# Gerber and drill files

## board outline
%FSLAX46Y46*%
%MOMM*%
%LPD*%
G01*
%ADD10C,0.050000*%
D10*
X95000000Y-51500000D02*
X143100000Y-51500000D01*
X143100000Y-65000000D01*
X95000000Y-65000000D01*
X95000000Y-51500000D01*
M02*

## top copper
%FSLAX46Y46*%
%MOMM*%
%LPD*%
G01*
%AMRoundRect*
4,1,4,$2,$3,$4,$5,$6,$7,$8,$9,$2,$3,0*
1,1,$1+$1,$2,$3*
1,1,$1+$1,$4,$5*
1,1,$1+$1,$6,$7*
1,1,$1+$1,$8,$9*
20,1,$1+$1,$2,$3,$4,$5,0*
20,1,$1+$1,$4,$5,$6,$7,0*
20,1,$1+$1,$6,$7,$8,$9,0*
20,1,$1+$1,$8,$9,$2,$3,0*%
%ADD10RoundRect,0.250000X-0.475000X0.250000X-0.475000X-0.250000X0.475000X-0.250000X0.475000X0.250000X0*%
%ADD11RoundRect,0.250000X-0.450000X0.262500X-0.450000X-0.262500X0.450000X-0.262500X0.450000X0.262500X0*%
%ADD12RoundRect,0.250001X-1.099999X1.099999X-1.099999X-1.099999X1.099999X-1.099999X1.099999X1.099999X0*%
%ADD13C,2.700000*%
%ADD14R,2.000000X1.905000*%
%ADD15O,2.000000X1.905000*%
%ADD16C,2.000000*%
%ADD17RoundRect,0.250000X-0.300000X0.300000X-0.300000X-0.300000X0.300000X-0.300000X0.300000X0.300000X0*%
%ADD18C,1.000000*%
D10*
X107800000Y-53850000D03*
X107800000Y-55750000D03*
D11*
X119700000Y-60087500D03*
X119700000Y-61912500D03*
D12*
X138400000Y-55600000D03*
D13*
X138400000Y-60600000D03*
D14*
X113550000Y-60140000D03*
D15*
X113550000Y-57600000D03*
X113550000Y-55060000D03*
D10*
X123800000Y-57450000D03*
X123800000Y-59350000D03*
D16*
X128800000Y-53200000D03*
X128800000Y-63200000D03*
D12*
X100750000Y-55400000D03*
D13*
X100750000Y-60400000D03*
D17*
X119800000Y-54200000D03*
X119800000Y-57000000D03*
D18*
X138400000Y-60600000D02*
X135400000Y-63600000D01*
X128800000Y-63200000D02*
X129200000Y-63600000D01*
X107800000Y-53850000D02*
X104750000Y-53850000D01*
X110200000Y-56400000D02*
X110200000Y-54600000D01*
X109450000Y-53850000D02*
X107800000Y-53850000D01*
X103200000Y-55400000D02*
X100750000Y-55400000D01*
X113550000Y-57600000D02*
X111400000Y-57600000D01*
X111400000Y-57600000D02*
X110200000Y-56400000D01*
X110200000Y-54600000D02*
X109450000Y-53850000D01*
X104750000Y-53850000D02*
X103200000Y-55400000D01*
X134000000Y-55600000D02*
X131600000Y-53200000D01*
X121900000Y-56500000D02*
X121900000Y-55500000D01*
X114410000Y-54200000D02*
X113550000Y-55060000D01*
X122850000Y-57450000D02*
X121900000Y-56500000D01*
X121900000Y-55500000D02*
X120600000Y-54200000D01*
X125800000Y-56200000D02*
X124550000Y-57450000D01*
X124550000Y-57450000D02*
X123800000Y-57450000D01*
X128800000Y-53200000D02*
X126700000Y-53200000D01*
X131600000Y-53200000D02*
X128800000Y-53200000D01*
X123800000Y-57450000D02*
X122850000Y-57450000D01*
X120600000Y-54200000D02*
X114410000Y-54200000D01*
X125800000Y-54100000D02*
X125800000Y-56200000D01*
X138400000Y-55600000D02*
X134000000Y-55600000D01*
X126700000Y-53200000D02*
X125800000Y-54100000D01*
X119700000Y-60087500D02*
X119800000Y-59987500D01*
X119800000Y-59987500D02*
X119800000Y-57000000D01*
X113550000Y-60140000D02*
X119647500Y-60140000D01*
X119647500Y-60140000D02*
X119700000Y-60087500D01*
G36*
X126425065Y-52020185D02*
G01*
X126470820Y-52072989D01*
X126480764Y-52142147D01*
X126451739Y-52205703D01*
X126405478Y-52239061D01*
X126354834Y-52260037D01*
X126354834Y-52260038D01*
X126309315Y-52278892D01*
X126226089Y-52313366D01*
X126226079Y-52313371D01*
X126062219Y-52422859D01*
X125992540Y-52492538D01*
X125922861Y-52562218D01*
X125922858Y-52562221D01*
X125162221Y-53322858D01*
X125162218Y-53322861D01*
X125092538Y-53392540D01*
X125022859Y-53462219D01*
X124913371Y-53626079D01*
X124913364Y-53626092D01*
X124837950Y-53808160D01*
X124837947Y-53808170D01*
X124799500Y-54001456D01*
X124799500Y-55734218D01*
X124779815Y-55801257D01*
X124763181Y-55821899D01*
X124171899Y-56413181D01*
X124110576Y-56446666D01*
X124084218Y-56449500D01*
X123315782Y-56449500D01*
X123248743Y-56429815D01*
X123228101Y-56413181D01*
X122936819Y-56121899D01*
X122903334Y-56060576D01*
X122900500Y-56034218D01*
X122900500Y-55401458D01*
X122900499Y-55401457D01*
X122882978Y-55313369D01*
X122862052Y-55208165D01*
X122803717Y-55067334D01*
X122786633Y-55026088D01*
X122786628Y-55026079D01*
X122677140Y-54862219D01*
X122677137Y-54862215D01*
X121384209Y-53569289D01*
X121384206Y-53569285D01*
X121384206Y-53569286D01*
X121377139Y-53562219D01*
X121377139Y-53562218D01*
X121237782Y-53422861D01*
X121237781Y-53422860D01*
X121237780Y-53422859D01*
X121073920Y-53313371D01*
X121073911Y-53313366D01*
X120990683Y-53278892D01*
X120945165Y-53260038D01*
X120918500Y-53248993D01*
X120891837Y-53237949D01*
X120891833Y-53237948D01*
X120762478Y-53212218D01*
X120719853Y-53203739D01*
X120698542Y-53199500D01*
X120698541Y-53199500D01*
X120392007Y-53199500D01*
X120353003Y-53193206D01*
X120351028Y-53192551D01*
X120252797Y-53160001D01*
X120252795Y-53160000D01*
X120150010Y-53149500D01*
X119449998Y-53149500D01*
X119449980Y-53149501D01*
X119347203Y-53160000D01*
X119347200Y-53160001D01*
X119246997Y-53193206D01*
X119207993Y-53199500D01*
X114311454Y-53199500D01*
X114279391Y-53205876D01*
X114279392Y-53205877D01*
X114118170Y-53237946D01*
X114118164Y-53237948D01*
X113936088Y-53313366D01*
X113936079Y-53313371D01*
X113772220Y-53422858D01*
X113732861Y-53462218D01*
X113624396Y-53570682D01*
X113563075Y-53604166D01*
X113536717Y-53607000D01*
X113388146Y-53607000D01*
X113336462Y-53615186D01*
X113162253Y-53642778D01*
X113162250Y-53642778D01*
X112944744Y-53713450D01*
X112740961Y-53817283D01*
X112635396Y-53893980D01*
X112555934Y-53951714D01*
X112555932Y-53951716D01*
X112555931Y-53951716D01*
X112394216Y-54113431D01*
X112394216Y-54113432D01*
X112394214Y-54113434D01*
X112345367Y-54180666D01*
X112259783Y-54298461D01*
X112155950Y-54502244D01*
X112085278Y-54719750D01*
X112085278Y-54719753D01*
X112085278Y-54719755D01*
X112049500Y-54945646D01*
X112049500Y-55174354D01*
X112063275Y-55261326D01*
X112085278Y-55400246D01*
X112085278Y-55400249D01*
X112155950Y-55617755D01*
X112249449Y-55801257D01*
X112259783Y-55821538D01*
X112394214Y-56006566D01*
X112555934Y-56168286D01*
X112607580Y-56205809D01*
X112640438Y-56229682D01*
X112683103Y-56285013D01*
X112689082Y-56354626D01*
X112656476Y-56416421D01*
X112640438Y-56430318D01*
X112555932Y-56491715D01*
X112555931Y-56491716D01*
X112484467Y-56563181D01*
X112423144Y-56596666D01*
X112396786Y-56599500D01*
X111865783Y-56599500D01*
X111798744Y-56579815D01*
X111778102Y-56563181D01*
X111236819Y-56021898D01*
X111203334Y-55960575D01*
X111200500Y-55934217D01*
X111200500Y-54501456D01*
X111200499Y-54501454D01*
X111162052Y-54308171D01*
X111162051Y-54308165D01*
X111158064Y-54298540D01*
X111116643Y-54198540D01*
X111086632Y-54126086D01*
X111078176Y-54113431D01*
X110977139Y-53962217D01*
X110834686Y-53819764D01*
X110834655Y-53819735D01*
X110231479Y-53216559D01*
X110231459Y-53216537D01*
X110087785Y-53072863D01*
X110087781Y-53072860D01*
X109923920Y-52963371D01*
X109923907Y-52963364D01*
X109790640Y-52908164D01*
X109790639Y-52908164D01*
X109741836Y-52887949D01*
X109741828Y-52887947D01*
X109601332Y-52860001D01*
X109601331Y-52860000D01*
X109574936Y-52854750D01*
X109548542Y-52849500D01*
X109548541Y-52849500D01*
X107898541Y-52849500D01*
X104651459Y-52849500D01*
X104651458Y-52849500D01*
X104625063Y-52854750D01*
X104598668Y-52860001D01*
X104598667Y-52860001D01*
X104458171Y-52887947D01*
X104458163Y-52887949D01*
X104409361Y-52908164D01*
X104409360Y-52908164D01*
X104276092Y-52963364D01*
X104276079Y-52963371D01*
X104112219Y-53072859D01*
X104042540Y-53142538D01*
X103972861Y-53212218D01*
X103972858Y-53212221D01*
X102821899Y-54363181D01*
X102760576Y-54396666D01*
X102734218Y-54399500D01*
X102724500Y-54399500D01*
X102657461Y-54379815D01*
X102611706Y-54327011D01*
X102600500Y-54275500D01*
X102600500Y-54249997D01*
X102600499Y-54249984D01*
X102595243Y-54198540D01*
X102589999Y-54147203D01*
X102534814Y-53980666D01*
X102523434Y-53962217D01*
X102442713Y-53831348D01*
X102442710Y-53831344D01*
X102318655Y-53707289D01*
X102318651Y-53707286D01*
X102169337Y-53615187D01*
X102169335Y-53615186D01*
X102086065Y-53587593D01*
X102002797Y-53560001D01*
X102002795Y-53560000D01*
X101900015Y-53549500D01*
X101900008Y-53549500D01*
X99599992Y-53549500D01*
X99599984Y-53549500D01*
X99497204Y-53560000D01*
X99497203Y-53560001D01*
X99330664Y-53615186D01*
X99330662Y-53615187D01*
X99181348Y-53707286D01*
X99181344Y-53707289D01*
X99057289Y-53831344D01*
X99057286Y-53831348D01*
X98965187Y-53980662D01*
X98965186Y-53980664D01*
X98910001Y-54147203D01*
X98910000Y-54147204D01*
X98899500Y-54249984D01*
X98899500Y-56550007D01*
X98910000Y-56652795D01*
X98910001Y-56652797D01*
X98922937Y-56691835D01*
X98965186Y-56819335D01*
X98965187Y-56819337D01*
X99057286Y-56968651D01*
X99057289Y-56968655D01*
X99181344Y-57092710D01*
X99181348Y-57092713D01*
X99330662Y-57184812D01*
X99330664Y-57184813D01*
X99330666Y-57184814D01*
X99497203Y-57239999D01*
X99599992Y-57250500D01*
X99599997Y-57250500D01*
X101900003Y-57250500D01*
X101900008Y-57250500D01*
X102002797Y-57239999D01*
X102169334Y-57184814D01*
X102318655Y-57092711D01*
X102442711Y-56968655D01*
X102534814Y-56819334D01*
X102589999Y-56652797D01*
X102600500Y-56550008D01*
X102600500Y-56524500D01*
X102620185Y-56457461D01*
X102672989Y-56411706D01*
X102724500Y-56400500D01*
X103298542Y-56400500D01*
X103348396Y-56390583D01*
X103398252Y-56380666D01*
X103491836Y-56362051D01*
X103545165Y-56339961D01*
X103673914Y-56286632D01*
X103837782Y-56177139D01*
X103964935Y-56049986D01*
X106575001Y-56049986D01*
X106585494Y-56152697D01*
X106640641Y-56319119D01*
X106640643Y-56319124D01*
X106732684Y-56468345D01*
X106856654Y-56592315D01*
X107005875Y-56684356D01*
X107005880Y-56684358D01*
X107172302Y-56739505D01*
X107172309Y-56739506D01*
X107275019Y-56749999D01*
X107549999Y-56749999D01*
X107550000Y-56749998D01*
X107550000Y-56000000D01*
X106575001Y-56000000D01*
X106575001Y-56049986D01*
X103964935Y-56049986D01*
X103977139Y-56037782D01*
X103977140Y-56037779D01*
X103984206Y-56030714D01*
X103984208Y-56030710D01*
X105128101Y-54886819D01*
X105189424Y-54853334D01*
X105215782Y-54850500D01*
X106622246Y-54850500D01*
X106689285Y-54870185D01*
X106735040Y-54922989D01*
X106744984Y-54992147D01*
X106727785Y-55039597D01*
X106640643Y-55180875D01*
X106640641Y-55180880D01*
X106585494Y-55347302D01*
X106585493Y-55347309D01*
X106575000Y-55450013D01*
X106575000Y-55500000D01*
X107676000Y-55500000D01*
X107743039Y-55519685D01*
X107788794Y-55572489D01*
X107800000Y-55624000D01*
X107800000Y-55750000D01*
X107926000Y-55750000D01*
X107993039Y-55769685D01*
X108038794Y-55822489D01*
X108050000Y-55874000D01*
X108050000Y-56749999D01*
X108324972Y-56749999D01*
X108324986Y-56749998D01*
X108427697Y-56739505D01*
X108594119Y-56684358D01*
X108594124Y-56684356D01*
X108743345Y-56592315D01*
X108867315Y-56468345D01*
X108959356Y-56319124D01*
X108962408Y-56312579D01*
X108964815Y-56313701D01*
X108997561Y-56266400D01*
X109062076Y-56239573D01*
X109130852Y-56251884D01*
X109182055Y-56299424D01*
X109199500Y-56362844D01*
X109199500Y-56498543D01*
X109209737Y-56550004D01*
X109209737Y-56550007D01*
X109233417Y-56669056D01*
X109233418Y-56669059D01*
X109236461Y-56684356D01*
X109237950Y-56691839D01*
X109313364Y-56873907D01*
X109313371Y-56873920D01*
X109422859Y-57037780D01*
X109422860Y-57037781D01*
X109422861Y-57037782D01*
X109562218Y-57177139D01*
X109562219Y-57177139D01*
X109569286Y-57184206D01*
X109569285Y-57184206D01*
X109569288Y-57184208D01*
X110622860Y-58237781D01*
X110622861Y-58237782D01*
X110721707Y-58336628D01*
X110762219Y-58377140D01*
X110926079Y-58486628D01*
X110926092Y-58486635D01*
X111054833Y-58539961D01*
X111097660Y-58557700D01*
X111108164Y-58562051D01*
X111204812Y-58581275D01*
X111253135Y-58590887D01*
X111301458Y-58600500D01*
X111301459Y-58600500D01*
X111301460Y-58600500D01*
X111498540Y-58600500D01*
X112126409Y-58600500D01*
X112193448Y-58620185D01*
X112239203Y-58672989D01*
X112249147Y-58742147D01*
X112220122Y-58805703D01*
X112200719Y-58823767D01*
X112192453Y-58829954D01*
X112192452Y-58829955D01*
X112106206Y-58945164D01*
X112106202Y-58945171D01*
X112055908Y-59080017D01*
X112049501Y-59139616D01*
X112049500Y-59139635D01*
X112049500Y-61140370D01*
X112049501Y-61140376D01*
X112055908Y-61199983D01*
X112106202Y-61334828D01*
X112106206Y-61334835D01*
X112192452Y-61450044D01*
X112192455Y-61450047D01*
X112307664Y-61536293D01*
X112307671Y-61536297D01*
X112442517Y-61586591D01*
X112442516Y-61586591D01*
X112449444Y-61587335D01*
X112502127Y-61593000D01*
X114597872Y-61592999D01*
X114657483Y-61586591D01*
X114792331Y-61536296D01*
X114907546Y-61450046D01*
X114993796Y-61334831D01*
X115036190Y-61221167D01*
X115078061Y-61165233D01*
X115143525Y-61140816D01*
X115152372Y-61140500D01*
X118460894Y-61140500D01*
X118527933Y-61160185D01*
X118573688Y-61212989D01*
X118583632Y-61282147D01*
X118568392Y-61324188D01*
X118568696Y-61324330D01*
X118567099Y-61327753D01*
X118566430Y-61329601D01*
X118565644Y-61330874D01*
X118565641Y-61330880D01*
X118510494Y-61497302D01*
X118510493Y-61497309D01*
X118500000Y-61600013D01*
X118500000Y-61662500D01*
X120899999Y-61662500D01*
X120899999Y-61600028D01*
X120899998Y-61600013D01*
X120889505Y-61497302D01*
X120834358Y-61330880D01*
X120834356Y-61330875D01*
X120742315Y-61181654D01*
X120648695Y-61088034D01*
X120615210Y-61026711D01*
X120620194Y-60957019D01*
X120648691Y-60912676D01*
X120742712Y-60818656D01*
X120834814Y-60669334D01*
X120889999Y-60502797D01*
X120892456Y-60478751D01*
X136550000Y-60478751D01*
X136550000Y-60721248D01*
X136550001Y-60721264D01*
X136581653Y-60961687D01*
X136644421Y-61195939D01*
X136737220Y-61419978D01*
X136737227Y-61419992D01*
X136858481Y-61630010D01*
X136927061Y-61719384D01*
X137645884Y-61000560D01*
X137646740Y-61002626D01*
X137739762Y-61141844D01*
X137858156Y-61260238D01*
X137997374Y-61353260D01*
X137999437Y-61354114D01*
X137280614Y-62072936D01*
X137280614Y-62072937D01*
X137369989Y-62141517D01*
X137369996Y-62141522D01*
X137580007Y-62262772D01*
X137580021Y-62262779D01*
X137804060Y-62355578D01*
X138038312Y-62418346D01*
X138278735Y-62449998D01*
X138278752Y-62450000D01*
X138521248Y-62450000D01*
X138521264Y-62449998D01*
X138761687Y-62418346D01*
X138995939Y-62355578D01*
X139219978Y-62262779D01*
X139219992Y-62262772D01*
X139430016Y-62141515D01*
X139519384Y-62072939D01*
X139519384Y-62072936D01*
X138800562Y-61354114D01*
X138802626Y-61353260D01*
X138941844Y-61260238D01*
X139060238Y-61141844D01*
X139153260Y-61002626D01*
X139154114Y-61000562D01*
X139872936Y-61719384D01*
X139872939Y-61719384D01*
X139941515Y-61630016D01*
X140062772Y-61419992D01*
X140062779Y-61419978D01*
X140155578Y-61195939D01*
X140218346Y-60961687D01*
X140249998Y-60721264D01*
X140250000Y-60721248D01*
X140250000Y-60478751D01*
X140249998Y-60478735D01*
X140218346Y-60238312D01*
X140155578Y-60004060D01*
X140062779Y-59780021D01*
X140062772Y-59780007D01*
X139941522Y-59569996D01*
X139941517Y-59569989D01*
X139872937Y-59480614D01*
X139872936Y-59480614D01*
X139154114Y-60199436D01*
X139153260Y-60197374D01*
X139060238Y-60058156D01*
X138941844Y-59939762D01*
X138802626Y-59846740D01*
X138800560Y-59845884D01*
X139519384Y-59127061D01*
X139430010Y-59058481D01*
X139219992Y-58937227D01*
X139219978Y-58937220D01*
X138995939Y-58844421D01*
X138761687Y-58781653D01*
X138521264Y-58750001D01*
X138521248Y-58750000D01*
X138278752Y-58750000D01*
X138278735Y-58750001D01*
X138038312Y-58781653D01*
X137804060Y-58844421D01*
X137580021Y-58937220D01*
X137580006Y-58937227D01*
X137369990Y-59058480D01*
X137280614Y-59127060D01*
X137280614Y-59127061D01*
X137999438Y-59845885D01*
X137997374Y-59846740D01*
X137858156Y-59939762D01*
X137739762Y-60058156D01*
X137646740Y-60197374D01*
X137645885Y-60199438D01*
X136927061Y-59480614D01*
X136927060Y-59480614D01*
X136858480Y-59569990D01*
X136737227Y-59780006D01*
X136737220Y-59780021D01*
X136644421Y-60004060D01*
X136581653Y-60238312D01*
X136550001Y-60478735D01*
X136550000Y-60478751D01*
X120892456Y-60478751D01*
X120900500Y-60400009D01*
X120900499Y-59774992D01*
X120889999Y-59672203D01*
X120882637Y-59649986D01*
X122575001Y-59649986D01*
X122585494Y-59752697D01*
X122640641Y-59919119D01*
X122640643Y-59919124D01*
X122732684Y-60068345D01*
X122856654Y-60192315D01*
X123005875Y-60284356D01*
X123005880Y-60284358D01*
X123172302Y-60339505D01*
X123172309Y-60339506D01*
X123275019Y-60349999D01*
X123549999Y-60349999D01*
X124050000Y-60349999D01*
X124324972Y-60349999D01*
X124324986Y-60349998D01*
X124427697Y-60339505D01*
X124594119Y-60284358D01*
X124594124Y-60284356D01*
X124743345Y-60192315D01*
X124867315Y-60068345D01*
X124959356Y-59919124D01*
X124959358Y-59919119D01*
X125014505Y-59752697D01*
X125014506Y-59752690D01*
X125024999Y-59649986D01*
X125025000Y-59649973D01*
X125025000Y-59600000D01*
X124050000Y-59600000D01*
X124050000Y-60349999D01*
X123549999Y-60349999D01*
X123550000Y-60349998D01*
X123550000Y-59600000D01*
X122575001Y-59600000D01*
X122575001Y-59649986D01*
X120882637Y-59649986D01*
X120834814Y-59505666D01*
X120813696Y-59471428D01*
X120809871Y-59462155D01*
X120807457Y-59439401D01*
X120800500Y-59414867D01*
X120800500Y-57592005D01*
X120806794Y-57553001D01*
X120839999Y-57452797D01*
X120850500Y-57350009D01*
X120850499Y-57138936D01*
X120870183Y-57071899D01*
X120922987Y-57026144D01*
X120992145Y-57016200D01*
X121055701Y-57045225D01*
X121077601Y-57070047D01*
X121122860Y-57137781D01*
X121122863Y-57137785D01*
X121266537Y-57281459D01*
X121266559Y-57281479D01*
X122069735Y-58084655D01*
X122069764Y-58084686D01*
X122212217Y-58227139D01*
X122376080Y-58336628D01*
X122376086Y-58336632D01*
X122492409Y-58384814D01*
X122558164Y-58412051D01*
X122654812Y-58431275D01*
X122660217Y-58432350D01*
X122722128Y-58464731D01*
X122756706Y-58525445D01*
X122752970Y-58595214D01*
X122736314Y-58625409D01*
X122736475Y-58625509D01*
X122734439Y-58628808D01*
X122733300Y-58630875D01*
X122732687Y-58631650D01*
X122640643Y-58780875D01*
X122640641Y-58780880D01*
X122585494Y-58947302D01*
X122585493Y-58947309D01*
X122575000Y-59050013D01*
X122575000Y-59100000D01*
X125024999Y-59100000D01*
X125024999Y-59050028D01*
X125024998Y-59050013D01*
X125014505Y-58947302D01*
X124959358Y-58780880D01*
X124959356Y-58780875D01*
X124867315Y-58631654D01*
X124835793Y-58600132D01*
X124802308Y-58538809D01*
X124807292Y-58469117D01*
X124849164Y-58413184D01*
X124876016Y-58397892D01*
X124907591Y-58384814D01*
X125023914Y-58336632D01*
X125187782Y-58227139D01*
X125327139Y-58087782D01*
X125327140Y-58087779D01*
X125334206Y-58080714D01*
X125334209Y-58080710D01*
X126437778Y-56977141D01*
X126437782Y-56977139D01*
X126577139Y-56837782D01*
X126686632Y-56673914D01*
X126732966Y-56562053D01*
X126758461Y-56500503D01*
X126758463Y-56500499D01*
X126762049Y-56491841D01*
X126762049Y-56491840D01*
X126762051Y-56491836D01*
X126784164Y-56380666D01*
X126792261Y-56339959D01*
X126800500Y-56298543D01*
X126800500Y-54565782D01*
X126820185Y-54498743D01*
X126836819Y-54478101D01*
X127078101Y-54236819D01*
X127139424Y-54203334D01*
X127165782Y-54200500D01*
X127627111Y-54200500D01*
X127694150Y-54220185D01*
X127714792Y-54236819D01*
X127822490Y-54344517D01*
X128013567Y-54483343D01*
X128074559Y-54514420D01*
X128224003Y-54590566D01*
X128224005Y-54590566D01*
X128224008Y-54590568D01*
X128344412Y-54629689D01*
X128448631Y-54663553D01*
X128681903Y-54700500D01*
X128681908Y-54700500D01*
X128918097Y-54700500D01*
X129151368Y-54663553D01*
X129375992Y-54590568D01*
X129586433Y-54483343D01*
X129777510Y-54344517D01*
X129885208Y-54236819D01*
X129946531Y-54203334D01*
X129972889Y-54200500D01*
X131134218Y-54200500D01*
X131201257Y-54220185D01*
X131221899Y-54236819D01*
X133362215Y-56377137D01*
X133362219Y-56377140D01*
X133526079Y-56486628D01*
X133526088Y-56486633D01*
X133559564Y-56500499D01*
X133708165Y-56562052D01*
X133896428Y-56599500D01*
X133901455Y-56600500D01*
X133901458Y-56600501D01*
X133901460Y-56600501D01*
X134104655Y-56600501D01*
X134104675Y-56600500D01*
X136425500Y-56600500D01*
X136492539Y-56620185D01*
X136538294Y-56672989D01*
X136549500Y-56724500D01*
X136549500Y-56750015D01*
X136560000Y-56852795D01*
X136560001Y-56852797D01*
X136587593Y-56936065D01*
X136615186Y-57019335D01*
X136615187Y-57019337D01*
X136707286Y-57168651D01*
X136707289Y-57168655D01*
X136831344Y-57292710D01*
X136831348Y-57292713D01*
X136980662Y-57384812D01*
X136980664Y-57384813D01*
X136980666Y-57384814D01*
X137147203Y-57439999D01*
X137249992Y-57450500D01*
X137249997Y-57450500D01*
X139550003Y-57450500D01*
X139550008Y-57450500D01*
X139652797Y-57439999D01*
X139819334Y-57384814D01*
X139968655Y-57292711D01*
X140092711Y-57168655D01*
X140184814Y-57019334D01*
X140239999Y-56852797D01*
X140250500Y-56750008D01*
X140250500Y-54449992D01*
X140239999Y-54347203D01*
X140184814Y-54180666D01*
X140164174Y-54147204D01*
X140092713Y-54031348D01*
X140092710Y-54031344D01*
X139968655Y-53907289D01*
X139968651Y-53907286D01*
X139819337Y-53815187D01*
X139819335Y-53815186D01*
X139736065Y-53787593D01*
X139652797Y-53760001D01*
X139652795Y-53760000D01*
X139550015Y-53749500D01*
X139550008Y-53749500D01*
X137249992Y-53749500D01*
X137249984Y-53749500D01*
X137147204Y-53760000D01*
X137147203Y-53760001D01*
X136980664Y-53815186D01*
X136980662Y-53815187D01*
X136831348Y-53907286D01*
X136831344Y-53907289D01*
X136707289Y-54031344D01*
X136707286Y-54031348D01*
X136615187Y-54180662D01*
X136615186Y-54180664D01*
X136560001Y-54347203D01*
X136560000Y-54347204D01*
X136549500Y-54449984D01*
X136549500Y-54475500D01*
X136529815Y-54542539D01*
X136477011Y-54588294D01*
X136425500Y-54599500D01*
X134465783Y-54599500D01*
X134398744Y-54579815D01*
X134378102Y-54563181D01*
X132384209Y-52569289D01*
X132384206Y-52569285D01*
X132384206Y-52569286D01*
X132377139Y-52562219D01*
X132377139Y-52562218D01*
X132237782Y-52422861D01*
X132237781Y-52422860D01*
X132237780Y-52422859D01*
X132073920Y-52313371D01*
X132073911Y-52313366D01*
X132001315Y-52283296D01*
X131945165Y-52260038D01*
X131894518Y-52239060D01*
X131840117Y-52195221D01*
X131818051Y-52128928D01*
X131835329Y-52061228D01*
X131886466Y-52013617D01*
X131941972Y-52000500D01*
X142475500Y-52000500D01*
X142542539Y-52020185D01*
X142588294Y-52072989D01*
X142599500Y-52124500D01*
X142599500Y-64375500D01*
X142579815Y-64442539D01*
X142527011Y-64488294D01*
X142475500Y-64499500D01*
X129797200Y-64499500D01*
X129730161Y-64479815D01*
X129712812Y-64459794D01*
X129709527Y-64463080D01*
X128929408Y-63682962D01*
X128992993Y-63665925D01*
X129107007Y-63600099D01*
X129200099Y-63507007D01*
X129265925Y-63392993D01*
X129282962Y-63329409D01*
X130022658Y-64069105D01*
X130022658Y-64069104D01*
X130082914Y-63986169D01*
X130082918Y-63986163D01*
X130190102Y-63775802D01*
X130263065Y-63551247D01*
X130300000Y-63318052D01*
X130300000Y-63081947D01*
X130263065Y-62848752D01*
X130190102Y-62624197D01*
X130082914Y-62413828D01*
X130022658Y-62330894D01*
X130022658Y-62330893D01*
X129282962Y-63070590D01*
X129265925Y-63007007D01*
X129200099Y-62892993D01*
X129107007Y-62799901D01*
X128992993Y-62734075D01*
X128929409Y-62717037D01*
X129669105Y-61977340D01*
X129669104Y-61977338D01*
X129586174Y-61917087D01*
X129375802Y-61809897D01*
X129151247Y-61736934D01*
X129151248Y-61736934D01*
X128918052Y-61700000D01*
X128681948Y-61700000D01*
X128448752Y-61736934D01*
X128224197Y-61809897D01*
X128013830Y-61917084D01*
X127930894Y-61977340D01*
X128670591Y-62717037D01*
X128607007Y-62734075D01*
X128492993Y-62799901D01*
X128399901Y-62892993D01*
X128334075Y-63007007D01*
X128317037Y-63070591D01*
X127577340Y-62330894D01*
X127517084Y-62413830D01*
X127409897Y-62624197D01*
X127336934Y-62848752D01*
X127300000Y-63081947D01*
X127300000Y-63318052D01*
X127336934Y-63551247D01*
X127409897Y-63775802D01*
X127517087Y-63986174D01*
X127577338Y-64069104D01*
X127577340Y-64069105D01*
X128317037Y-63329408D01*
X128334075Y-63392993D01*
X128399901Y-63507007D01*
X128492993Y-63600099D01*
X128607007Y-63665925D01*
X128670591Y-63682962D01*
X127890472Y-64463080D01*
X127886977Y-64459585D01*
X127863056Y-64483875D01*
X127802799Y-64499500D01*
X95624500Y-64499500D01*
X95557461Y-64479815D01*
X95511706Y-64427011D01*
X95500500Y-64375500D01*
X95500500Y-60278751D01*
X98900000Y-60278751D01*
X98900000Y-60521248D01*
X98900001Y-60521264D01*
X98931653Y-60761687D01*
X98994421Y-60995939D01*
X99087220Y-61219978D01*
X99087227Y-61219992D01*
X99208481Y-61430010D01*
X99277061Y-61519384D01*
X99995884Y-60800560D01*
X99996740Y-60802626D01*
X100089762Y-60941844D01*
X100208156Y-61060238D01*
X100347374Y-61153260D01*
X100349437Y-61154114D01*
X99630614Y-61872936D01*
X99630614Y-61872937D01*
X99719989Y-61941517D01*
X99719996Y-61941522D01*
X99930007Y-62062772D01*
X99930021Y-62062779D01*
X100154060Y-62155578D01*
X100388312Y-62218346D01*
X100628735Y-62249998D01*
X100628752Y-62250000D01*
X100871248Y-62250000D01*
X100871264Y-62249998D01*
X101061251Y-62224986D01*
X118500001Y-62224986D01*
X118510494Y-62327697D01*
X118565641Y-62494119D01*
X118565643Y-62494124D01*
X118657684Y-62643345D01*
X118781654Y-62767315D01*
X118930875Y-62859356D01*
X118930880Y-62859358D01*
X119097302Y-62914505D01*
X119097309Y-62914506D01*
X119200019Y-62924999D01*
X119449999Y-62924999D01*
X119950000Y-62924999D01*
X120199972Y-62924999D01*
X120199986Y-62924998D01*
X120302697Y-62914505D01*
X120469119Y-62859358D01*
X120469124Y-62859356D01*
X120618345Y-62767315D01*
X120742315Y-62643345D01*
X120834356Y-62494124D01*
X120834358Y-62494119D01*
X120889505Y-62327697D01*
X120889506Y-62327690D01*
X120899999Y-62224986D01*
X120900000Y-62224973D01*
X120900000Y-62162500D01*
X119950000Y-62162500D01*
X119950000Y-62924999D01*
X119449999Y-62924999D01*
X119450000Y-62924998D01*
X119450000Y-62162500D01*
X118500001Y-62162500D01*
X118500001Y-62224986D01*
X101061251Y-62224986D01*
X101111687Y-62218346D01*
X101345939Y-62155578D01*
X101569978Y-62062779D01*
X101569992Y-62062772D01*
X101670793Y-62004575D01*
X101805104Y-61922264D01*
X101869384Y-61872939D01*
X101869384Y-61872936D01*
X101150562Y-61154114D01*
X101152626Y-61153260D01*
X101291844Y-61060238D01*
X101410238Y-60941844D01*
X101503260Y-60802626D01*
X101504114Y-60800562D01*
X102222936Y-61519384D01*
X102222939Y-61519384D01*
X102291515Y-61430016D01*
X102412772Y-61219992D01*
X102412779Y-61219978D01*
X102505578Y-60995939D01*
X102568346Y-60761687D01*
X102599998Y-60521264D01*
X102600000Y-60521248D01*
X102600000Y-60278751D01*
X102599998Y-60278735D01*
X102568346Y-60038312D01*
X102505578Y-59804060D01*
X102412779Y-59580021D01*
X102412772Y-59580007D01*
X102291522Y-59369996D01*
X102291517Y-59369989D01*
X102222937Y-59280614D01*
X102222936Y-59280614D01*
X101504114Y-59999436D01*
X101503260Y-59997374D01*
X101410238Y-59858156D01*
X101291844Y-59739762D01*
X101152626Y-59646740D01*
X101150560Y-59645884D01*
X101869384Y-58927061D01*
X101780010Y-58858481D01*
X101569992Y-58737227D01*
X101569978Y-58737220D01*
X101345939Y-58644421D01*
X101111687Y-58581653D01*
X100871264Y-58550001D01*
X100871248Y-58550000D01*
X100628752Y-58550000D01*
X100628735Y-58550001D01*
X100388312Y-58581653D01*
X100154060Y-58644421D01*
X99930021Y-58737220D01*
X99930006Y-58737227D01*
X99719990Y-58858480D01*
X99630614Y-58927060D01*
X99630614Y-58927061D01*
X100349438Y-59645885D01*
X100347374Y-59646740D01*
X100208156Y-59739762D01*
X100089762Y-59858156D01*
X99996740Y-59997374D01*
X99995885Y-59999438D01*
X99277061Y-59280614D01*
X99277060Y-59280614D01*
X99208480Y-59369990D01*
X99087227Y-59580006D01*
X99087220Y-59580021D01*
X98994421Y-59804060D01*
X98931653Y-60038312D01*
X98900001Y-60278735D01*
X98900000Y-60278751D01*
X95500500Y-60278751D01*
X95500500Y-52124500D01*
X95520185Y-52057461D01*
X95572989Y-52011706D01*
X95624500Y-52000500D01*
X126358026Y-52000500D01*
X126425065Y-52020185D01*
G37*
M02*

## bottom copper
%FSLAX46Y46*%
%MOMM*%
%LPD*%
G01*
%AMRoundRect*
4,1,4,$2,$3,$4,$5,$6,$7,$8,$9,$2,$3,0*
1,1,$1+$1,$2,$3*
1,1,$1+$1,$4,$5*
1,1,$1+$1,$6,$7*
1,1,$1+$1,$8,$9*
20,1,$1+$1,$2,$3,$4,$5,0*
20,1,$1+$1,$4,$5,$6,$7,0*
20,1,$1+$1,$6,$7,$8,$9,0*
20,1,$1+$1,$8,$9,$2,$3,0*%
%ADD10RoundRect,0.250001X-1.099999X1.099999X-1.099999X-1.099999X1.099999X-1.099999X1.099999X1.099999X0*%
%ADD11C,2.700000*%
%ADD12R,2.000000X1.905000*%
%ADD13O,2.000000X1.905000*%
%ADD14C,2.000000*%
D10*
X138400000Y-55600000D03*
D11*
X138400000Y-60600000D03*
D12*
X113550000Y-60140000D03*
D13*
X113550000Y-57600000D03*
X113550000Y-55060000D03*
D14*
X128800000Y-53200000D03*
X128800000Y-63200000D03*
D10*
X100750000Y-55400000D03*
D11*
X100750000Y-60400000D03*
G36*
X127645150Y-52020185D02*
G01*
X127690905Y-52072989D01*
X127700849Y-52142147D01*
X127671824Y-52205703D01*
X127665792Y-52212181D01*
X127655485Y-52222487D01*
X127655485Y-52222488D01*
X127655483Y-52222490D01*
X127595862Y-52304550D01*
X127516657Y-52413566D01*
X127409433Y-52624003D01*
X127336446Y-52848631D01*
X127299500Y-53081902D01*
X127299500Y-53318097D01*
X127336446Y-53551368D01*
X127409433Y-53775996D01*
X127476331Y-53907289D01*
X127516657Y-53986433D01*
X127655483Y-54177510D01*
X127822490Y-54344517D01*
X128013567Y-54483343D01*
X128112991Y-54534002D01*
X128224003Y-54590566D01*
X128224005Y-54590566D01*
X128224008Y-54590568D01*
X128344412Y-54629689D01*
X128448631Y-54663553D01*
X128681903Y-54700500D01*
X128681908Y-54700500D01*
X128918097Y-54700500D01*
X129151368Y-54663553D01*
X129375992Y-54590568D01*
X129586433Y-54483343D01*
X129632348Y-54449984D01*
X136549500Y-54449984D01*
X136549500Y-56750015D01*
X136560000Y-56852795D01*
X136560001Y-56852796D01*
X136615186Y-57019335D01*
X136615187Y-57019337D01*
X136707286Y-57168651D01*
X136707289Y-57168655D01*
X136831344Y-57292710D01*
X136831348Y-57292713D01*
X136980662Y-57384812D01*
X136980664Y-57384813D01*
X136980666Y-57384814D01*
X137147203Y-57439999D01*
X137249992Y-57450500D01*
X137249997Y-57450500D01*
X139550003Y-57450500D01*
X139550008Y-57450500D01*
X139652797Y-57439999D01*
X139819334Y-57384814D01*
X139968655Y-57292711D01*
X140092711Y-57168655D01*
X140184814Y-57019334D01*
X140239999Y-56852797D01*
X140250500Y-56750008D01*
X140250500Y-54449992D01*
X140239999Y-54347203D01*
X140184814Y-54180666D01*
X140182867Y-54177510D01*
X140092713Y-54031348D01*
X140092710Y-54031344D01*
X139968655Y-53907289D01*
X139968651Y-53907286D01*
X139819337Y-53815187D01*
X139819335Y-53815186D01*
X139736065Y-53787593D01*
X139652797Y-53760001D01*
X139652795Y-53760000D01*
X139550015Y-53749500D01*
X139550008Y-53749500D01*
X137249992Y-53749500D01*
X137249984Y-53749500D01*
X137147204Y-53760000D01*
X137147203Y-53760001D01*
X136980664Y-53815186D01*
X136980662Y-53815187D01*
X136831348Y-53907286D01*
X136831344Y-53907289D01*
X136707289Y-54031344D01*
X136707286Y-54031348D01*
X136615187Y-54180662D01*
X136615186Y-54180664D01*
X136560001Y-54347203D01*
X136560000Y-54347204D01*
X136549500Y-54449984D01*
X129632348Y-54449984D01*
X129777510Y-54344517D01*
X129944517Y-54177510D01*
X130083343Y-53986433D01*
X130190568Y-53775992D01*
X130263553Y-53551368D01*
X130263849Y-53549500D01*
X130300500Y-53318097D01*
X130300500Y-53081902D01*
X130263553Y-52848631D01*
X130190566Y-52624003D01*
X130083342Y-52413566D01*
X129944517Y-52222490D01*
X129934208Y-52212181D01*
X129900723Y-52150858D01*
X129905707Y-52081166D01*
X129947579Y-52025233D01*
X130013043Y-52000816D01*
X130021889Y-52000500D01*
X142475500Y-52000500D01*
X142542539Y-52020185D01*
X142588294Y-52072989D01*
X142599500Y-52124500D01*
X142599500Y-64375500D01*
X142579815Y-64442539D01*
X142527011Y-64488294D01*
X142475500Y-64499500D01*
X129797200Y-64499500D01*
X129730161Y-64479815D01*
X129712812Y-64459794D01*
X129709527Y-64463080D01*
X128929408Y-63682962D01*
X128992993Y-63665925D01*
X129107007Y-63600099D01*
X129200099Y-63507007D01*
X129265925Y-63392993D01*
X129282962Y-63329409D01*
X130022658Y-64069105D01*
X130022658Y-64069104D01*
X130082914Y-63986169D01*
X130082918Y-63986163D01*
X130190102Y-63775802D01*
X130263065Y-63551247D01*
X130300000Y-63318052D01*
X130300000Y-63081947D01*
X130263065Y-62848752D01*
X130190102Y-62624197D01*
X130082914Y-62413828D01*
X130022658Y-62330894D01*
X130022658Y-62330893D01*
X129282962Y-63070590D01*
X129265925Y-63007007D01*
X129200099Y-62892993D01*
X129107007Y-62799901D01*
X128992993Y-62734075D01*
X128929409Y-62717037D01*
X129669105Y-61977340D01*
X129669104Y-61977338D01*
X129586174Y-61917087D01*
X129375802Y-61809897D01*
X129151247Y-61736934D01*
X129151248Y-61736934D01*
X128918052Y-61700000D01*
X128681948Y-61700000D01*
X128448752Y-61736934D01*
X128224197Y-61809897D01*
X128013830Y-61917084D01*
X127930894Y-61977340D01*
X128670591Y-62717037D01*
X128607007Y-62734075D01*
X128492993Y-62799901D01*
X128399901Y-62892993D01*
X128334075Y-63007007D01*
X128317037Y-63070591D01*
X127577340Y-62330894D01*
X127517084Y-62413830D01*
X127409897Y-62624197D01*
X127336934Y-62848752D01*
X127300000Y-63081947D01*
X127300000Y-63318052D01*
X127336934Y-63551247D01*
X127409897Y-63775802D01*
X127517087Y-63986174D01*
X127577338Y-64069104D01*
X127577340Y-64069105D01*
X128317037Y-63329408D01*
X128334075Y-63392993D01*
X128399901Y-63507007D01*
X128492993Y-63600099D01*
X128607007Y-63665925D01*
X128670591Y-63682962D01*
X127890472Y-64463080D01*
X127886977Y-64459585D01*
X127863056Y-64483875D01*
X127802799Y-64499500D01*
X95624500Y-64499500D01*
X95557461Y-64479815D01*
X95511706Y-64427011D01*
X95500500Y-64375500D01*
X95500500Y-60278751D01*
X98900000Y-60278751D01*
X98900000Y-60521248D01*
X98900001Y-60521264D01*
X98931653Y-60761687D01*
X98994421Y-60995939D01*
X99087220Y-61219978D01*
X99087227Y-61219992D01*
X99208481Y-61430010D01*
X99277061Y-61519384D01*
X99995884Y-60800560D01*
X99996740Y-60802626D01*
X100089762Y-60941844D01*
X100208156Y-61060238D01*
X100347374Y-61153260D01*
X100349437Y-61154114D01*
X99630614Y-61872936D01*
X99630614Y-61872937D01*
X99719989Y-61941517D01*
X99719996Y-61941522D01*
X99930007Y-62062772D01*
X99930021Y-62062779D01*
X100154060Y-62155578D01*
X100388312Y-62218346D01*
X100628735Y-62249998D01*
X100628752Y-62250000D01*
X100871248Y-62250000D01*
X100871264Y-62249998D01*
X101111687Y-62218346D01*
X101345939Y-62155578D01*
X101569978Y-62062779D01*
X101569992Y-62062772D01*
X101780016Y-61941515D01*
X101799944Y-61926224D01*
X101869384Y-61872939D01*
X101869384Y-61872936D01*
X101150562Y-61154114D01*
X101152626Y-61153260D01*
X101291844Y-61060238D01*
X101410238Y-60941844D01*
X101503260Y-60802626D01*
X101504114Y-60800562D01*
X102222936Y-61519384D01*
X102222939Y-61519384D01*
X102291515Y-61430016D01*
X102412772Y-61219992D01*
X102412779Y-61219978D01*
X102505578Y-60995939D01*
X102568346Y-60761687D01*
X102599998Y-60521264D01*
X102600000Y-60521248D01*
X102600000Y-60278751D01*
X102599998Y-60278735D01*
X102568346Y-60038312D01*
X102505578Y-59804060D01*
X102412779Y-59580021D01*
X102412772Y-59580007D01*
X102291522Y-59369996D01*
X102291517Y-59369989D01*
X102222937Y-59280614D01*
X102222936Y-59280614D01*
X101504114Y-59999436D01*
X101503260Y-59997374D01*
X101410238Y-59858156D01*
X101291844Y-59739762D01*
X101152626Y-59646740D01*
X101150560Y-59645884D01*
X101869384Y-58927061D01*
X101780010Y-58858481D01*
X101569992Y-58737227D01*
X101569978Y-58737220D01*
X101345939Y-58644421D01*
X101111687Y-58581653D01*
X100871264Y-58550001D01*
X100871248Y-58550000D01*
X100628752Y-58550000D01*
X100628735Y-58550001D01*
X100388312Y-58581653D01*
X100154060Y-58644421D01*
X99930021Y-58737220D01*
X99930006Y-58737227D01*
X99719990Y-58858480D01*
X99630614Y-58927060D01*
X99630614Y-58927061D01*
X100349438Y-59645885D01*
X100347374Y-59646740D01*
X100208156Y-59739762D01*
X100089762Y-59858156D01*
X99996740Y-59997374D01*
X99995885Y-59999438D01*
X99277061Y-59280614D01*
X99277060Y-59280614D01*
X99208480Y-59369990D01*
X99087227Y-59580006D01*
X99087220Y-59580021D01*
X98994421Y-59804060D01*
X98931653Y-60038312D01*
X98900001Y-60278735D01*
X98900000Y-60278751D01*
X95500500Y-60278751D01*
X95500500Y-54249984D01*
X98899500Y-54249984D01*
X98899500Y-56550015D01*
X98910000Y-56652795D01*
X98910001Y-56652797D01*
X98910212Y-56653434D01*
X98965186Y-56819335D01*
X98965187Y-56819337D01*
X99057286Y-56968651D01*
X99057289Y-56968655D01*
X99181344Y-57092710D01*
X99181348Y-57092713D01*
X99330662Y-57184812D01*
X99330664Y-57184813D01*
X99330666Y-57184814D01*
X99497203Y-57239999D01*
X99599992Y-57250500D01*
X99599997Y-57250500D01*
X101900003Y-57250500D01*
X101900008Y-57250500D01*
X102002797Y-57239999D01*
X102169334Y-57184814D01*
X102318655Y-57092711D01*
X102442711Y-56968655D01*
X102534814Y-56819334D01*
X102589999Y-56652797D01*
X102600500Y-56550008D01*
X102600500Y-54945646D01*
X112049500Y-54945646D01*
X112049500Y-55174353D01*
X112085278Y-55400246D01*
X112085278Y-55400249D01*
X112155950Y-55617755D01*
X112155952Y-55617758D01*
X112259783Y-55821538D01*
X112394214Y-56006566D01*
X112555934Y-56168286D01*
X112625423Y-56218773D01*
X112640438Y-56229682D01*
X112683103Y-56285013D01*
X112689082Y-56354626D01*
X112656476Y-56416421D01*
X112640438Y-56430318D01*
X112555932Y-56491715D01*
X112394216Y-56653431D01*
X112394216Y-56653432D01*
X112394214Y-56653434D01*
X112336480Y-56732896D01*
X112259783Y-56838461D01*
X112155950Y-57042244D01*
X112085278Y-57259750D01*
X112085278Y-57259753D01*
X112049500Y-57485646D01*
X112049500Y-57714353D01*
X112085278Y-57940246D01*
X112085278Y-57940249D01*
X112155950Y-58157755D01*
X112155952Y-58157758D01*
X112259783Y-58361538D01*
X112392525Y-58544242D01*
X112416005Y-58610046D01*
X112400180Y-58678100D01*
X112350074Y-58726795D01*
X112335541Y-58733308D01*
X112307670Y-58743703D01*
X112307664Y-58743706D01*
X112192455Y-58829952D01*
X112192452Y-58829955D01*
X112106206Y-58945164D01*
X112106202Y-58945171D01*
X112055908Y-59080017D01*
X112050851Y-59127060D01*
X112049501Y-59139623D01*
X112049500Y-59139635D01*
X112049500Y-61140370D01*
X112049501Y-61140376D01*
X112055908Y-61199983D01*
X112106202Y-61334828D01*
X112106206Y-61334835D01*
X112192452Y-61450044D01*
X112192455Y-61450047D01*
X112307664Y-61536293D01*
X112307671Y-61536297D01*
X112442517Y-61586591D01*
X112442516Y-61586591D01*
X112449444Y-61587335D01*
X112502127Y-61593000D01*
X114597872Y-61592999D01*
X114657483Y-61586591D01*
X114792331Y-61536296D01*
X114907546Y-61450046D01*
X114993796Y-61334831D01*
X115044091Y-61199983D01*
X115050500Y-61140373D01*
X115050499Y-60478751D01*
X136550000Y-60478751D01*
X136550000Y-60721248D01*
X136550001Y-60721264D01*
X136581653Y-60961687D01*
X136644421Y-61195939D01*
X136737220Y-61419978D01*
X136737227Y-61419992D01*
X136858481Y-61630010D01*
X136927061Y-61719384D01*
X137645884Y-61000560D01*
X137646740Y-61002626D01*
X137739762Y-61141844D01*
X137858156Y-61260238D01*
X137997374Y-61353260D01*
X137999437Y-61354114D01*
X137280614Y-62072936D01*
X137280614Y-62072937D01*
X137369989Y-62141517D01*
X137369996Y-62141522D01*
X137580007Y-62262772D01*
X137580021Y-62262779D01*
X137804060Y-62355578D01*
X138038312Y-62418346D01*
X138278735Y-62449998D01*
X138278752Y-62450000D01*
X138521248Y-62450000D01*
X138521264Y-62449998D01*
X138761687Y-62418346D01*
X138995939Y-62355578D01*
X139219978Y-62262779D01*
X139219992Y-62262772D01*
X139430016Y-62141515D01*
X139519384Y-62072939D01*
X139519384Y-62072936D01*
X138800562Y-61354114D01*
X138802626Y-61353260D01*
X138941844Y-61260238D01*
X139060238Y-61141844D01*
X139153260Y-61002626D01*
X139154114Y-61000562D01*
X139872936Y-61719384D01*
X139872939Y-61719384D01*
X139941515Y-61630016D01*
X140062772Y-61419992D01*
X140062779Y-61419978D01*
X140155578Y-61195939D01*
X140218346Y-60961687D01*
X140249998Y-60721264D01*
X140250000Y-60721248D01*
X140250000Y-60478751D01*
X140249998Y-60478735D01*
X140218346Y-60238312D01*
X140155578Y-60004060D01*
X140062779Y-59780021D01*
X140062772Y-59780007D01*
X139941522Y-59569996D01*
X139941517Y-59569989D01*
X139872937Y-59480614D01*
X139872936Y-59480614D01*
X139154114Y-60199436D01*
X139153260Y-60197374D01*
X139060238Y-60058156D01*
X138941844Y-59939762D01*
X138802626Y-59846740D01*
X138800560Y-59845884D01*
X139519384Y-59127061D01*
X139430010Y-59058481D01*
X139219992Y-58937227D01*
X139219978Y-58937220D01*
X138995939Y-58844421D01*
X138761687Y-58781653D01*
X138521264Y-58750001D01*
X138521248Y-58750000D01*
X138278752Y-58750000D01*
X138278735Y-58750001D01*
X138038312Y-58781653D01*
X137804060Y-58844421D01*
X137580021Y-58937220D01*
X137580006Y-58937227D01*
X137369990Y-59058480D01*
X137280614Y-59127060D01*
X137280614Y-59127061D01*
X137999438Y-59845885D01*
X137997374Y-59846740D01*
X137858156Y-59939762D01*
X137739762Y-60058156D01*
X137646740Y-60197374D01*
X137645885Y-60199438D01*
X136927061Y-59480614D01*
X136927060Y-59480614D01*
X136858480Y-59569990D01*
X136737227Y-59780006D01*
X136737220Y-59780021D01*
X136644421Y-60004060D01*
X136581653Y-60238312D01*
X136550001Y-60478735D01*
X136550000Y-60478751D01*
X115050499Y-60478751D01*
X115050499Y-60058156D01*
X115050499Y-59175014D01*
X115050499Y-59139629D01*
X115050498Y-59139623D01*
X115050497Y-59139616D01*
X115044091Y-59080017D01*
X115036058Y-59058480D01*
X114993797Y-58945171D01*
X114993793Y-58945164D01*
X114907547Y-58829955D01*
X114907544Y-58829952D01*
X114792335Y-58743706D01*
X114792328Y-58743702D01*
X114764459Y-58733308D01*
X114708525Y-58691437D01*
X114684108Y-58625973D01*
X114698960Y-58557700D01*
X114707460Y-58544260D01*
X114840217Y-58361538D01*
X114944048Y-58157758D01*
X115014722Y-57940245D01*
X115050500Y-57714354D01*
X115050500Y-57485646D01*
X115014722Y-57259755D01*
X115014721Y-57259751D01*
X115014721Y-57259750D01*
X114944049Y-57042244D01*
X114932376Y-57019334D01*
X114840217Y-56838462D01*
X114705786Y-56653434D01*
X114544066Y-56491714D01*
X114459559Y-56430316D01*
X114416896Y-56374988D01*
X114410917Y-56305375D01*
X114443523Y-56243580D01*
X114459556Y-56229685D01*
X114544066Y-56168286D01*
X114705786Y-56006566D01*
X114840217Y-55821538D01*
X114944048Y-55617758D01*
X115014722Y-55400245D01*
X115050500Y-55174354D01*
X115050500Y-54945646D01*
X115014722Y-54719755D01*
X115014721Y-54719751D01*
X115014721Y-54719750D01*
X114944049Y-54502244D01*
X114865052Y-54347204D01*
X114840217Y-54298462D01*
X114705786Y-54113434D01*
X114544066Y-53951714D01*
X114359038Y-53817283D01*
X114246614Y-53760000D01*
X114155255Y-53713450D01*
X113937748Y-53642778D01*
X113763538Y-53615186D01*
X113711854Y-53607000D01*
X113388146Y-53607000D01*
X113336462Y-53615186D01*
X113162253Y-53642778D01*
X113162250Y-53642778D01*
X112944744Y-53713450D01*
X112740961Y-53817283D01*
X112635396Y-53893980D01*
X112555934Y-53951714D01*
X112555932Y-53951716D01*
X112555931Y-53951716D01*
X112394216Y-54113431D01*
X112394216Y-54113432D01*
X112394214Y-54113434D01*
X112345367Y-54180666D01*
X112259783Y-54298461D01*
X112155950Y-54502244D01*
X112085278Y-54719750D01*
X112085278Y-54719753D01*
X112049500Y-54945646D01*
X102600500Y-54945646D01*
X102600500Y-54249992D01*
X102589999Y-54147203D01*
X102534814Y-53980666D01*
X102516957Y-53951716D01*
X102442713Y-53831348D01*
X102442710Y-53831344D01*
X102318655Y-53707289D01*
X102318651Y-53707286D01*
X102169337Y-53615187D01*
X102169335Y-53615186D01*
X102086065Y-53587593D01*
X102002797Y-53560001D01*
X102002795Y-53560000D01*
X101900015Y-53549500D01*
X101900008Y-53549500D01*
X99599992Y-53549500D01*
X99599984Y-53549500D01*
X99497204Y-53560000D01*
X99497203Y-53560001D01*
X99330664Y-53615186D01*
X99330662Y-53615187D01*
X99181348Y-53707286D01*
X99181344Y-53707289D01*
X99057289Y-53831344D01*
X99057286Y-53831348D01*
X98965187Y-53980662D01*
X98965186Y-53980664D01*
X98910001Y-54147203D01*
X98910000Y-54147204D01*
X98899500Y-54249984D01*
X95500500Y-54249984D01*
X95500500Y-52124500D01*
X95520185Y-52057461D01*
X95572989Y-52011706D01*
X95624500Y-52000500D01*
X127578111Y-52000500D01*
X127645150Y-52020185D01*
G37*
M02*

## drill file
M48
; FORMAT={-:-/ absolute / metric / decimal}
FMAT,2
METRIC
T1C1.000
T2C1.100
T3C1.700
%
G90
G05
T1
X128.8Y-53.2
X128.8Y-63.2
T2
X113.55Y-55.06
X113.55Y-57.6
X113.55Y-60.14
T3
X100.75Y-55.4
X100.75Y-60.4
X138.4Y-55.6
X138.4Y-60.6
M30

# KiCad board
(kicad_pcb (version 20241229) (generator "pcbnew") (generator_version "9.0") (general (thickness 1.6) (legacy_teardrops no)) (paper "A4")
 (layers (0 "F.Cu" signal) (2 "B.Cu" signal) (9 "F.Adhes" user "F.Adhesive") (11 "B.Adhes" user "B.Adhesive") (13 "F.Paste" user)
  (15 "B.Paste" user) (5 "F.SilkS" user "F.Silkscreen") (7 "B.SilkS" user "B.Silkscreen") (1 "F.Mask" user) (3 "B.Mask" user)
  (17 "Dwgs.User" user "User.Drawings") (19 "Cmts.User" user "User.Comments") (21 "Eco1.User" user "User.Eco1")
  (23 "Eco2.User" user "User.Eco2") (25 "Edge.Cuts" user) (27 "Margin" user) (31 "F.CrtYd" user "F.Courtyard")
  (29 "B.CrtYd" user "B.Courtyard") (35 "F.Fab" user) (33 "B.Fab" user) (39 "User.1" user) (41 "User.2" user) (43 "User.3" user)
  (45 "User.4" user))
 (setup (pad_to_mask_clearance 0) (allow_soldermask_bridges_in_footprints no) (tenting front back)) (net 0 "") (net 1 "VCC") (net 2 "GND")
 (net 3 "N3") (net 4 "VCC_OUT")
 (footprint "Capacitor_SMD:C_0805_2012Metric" (layer "F.Cu") (at 107.8 54.8 -90)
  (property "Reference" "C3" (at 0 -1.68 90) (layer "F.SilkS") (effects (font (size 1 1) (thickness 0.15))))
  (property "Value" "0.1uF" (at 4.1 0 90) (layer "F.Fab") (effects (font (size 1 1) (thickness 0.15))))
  (pad "1" smd roundrect (at -0.95 0 270) (size 1 1.45) (layers "F.Cu" "F.Mask" "F.Paste") (roundrect_rratio 0.25) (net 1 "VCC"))
  (pad "2" smd roundrect (at 0.95 0 270) (size 1 1.45) (layers "F.Cu" "F.Mask" "F.Paste") (roundrect_rratio 0.25) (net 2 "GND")))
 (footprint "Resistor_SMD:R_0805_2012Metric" (layer "F.Cu") (at 119.7 61 -90)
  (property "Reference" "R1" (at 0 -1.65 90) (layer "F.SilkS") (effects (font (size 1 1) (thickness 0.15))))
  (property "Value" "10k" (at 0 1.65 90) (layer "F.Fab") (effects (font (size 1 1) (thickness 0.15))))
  (pad "1" smd roundrect (at -0.9125 0 270) (size 1.025 1.4) (layers "F.Cu" "F.Mask" "F.Paste") (roundrect_rratio 0.243902) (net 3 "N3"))
  (pad "2" smd roundrect (at 0.9125 0 270) (size 1.025 1.4) (layers "F.Cu" "F.Mask" "F.Paste") (roundrect_rratio 0.243902) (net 2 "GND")))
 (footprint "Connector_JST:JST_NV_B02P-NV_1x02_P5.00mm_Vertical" (layer "F.Cu") (at 138.4 55.6 -90)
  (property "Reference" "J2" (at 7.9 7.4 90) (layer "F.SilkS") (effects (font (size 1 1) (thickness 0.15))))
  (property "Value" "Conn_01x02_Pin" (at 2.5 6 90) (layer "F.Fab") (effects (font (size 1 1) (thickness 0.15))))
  (pad "1" thru_hole roundrect (at 0 0 270) (size 2.7 2.7) (drill 1.7) (layers "*.Cu" "*.Mask") (remove_unused_layers no)
   (roundrect_rratio 0.092593) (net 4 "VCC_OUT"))
  (pad "2" thru_hole circle (at 5 0 270) (size 2.7 2.7) (drill 1.7) (layers "*.Cu" "*.Mask") (remove_unused_layers no) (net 2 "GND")))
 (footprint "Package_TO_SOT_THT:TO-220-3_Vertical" (layer "F.Cu") (at 113.55 60.14 90)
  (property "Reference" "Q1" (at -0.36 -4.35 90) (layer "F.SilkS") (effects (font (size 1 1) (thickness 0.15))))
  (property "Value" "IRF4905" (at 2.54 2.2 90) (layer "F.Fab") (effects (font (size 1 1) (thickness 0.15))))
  (pad "1" thru_hole rect (at 0 0 90) (size 1.905 2) (drill 1.1) (layers "*.Cu" "*.Mask") (remove_unused_layers no) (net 3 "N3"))
  (pad "2" thru_hole oval (at 2.54 0 90) (size 1.905 2) (drill 1.1) (layers "*.Cu" "*.Mask") (remove_unused_layers no) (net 1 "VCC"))
  (pad "3" thru_hole oval (at 5.08 0 90) (size 1.905 2) (drill 1.1) (layers "*.Cu" "*.Mask") (remove_unused_layers no) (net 4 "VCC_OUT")))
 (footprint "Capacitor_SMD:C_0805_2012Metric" (layer "F.Cu") (at 123.8 58.4 -90)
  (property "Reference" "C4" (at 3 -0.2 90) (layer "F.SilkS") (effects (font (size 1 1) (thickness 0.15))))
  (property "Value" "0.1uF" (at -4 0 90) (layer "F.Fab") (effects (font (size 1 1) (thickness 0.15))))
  (pad "1" smd roundrect (at -0.95 0 270) (size 1 1.45) (layers "F.Cu" "F.Mask" "F.Paste") (roundrect_rratio 0.25) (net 4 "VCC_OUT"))
  (pad "2" smd roundrect (at 0.95 0 270) (size 1 1.45) (layers "F.Cu" "F.Mask" "F.Paste") (roundrect_rratio 0.25) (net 2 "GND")))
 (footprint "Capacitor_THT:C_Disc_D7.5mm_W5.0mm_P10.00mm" (layer "F.Cu") (at 128.8 53.2 -90)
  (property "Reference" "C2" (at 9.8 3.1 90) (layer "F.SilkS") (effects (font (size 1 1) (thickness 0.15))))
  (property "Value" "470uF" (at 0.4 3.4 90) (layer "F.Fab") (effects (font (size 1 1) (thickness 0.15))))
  (pad "1" thru_hole circle (at 0 0 270) (size 2 2) (drill 1) (layers "*.Cu" "*.Mask") (remove_unused_layers no) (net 4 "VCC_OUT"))
  (pad "2" thru_hole circle (at 10 0 270) (size 2 2) (drill 1) (layers "*.Cu" "*.Mask") (remove_unused_layers no) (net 2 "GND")))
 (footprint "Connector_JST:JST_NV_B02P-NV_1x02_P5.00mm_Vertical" (layer "F.Cu") (at 100.75 55.4 -90)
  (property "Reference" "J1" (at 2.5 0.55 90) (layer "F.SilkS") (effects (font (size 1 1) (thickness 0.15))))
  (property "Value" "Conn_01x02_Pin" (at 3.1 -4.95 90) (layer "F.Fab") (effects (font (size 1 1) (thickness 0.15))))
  (pad "1" thru_hole roundrect (at 0 0 270) (size 2.7 2.7) (drill 1.7) (layers "*.Cu" "*.Mask") (remove_unused_layers no)
   (roundrect_rratio 0.092593) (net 1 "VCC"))
  (pad "2" thru_hole circle (at 5 0 270) (size 2.7 2.7) (drill 1.7) (layers "*.Cu" "*.Mask") (remove_unused_layers no) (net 2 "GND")))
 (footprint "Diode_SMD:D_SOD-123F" (layer "F.Cu") (at 119.8 55.6 -90)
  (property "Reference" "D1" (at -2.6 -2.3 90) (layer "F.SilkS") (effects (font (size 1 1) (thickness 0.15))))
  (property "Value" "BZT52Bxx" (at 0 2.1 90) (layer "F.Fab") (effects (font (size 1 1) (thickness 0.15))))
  (pad "1" smd roundrect (at -1.4 0 270) (size 1.1 1.1) (layers "F.Cu" "F.Mask" "F.Paste") (roundrect_rratio 0.2272727273) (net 4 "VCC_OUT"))
  (pad "2" smd roundrect (at 1.4 0 270) (size 1.1 1.1) (layers "F.Cu" "F.Mask" "F.Paste") (roundrect_rratio 0.2272727273) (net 3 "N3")))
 (gr_rect (start 95 51.5) (end 143.1 65) (stroke (width 0.05) (type default)) (fill no) (layer "Edge.Cuts"))
 (segment (start 138.4 60.6) (end 135.4 63.6) (width 1) (layer "F.Cu") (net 2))
 (segment (start 128.8 63.2) (end 129.2 63.6) (width 1) (layer "F.Cu") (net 2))
 (segment (start 107.8 53.85) (end 104.75 53.85) (width 1) (layer "F.Cu") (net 1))
 (segment (start 110.2 56.4) (end 110.2 54.6) (width 1) (layer "F.Cu") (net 1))
 (segment (start 109.45 53.85) (end 107.8 53.85) (width 1) (layer "F.Cu") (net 1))
 (segment (start 103.2 55.4) (end 100.75 55.4) (width 1) (layer "F.Cu") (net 1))
 (segment (start 113.55 57.6) (end 111.4 57.6) (width 1) (layer "F.Cu") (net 1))
 (segment (start 111.4 57.6) (end 110.2 56.4) (width 1) (layer "F.Cu") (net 1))
 (segment (start 110.2 54.6) (end 109.45 53.85) (width 1) (layer "F.Cu") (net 1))
 (segment (start 104.75 53.85) (end 103.2 55.4) (width 1) (layer "F.Cu") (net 1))
 (segment (start 134 55.6) (end 131.6 53.2) (width 1) (layer "F.Cu") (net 4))
 (segment (start 121.9 56.5) (end 121.9 55.5) (width 1) (layer "F.Cu") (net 4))
 (segment (start 114.41 54.2) (end 113.55 55.06) (width 1) (layer "F.Cu") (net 4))
 (segment (start 122.85 57.45) (end 121.9 56.5) (width 1) (layer "F.Cu") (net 4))
 (segment (start 121.9 55.5) (end 120.6 54.2) (width 1) (layer "F.Cu") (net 4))
 (segment (start 125.8 56.2) (end 124.55 57.45) (width 1) (layer "F.Cu") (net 4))
 (segment (start 124.55 57.45) (end 123.8 57.45) (width 1) (layer "F.Cu") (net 4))
 (segment (start 128.8 53.2) (end 126.7 53.2) (width 1) (layer "F.Cu") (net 4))
 (segment (start 131.6 53.2) (end 128.8 53.2) (width 1) (layer "F.Cu") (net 4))
 (segment (start 123.8 57.45) (end 122.85 57.45) (width 1) (layer "F.Cu") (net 4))
 (segment (start 120.6 54.2) (end 114.41 54.2) (width 1) (layer "F.Cu") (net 4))
 (segment (start 125.8 54.1) (end 125.8 56.2) (width 1) (layer "F.Cu") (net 4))
 (segment (start 138.4 55.6) (end 134 55.6) (width 1) (layer "F.Cu") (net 4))
 (segment (start 126.7 53.2) (end 125.8 54.1) (width 1) (layer "F.Cu") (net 4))
 (segment (start 119.7 60.0875) (end 119.8 59.9875) (width 1) (layer "F.Cu") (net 3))
 (segment (start 119.8 59.9875) (end 119.8 57) (width 1) (layer "F.Cu") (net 3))
 (segment (start 113.55 60.14) (end 119.6475 60.14) (width 1) (layer "F.Cu") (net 3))
 (segment (start 119.6475 60.14) (end 119.7 60.0875) (width 1) (layer "F.Cu") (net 3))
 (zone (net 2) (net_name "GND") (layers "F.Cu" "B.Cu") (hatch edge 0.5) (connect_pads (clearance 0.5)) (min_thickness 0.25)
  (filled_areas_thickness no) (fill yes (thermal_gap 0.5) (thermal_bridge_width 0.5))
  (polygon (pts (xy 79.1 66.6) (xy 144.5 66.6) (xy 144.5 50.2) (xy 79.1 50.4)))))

